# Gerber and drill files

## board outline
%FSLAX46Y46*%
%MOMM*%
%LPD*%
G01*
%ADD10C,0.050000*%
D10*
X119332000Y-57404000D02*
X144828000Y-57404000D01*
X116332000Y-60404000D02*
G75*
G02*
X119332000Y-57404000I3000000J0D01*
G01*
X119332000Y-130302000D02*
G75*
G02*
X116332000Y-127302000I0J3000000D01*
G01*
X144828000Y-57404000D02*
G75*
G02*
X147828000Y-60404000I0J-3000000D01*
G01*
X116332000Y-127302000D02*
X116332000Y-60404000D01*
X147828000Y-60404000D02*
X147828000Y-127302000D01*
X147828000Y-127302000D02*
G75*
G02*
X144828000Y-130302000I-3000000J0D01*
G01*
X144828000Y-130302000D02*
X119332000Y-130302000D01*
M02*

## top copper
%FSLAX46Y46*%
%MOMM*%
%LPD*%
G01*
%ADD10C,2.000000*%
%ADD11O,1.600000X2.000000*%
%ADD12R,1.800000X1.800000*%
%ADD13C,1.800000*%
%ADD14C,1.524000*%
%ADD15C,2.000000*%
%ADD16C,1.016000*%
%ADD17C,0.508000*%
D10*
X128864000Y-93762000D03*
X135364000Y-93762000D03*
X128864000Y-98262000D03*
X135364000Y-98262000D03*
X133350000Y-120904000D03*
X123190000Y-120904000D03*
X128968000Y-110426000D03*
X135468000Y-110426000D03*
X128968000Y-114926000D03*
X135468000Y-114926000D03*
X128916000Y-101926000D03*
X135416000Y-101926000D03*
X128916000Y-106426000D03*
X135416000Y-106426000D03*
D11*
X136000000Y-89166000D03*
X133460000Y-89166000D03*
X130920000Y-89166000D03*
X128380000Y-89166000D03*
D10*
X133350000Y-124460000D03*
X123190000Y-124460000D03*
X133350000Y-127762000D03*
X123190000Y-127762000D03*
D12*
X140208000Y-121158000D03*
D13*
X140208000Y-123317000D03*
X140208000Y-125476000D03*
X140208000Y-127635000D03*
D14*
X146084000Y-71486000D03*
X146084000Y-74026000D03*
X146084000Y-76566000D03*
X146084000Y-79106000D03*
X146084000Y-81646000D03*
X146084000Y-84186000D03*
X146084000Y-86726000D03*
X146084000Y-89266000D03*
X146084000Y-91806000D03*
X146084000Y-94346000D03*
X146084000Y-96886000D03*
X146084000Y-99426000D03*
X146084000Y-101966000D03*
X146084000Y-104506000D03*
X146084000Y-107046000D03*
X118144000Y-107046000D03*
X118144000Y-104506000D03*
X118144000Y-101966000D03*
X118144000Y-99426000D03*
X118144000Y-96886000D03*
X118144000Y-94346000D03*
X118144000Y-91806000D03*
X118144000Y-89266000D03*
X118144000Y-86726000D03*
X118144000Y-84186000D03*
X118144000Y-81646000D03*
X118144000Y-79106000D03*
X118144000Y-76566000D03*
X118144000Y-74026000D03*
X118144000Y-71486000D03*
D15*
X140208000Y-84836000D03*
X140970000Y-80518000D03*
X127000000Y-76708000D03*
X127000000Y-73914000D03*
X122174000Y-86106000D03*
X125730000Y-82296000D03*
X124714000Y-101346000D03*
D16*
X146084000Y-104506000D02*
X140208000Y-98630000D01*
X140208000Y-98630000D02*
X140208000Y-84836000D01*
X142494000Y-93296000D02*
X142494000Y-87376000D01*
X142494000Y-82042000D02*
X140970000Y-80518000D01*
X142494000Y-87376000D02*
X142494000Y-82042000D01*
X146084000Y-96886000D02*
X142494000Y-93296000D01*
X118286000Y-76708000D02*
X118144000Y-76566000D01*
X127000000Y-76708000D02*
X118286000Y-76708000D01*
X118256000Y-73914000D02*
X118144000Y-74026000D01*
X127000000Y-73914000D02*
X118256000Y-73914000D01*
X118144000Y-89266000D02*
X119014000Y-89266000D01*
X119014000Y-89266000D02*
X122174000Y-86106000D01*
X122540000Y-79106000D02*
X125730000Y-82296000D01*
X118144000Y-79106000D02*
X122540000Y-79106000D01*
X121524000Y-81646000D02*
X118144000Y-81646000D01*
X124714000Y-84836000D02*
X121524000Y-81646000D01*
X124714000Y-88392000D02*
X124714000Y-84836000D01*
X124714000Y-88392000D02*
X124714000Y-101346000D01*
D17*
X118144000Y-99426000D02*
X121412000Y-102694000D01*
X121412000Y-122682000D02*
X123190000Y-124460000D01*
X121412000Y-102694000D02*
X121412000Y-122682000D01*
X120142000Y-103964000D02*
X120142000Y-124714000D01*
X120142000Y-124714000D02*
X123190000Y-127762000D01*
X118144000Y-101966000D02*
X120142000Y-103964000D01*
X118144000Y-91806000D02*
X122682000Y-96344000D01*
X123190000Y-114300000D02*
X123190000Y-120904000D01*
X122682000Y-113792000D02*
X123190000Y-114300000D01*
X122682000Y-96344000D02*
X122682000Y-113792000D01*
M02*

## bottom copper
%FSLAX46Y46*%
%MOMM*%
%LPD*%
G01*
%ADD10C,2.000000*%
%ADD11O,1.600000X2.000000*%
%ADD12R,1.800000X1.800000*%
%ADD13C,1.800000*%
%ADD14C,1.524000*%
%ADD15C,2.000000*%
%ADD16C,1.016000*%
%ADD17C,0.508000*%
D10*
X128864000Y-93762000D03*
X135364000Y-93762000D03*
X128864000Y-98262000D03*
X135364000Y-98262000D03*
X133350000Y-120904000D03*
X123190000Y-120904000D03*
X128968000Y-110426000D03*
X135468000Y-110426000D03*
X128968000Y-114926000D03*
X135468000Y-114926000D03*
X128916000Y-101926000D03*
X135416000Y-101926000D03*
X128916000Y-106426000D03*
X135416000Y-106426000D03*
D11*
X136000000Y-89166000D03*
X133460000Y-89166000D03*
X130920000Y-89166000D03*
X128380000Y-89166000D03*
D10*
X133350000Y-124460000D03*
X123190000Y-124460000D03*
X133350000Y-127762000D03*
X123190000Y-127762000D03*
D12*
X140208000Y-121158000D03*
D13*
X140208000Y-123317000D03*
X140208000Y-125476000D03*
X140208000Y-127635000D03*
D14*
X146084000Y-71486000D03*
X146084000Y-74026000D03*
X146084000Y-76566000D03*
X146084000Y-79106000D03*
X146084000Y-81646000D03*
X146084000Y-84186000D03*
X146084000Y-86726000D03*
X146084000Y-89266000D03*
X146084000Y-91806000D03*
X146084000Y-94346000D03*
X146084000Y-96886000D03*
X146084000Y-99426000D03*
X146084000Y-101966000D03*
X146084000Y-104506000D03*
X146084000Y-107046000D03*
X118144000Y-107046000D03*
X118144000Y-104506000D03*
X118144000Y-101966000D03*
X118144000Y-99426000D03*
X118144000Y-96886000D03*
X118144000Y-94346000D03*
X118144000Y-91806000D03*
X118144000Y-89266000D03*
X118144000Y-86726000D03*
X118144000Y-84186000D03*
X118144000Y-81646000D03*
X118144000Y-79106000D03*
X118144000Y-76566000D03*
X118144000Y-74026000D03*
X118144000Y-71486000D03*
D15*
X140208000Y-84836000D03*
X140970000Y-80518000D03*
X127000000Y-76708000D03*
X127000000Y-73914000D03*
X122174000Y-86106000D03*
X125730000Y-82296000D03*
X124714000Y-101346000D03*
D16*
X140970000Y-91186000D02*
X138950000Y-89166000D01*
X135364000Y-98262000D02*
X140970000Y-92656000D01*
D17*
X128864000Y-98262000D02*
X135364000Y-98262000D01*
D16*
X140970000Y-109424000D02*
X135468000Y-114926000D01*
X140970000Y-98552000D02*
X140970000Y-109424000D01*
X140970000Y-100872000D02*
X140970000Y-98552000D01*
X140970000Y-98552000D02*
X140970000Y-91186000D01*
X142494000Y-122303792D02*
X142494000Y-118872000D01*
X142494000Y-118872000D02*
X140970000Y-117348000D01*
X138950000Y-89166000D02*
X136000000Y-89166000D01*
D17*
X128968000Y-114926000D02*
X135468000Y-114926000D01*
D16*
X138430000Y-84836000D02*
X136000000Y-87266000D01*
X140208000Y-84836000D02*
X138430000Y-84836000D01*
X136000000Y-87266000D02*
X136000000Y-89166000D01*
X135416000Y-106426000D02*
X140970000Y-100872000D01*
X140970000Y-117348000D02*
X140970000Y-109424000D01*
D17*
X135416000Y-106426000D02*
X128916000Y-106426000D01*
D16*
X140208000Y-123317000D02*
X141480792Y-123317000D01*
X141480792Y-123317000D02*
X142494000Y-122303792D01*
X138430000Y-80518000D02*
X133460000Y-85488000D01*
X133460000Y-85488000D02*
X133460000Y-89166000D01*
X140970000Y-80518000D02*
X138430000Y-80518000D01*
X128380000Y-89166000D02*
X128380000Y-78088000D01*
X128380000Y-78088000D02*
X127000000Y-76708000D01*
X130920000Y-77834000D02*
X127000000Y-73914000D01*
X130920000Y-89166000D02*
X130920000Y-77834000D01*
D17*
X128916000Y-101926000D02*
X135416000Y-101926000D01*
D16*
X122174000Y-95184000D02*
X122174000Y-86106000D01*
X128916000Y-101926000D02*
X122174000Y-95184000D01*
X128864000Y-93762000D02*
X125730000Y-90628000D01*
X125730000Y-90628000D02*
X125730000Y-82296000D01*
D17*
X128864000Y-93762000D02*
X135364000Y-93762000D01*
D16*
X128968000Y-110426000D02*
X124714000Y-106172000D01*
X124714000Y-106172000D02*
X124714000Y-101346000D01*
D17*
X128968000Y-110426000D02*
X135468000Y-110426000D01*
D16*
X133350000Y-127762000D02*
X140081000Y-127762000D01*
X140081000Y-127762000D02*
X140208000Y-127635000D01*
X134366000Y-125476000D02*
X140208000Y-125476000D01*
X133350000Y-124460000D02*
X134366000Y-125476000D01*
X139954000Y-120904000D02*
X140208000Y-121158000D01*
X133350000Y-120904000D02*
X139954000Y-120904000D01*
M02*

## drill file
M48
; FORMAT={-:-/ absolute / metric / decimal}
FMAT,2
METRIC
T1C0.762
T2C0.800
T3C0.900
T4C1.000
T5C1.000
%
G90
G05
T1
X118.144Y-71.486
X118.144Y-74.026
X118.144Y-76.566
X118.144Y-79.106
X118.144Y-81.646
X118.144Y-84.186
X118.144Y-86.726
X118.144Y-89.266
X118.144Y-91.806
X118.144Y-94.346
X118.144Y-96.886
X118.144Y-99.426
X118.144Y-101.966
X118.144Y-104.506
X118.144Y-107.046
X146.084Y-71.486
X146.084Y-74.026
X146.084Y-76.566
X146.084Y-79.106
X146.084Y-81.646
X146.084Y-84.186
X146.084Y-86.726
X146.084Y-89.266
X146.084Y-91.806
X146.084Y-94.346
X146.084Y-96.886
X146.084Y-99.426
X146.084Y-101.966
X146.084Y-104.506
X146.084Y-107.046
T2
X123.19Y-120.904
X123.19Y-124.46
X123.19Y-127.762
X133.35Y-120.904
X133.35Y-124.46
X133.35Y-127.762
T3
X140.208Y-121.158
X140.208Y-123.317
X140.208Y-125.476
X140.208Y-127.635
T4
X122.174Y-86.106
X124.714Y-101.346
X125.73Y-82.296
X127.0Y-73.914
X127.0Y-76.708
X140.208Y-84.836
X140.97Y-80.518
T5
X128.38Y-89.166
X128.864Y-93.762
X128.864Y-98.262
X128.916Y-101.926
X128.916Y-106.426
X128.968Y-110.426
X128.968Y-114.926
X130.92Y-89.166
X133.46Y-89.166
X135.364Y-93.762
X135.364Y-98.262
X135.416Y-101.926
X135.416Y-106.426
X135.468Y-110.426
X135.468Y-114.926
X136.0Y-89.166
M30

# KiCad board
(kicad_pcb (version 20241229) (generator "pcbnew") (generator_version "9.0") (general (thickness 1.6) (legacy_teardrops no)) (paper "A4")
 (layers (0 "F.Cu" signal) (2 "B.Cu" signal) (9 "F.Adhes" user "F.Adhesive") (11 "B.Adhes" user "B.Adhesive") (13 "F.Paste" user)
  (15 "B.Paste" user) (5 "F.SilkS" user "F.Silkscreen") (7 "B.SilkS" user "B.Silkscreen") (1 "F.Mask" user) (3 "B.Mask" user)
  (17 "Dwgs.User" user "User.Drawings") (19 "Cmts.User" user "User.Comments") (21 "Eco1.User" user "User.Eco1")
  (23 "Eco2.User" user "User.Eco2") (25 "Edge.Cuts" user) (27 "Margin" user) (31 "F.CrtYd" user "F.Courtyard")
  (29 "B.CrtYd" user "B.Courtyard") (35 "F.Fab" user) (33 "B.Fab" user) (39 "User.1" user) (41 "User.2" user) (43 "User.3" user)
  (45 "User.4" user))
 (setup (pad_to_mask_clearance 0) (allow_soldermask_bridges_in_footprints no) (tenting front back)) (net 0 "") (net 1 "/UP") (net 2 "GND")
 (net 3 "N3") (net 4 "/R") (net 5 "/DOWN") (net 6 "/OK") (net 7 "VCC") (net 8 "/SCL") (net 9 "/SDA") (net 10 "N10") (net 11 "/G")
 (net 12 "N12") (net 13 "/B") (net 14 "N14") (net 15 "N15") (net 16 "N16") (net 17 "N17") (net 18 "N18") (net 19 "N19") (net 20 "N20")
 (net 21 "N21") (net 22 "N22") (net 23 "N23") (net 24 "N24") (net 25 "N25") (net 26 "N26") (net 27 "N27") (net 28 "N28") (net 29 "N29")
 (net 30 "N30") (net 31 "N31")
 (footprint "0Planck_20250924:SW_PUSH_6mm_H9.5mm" (layer "F.Cu") (at 128.864 93.762)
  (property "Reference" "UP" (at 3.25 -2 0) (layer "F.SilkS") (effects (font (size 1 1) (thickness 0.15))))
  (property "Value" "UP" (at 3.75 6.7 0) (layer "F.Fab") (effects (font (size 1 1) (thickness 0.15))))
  (pad "1" thru_hole circle (at 0 0) (size 2 2) (drill 1) (layers "*.Cu" "*.Mask") (remove_unused_layers no) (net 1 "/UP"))
  (pad "1" thru_hole circle (at 6.5 0) (size 2 2) (drill 1) (layers "*.Cu" "*.Mask") (remove_unused_layers no) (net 1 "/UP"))
  (pad "2" thru_hole circle (at 0 4.5) (size 2 2) (drill 1) (layers "*.Cu" "*.Mask") (remove_unused_layers no) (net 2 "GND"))
  (pad "2" thru_hole circle (at 6.5 4.5) (size 2 2) (drill 1) (layers "*.Cu" "*.Mask") (remove_unused_layers no) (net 2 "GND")))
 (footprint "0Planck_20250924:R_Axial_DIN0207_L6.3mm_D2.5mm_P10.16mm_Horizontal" (layer "F.Cu") (at 133.35 120.904 180)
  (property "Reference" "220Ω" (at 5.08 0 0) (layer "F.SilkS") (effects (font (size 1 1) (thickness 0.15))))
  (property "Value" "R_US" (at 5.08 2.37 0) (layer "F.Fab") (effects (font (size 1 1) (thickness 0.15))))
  (pad "1" thru_hole circle (at 0 0 180) (size 2 2) (drill 0.8) (layers "*.Cu" "*.Mask") (remove_unused_layers no) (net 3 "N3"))
  (pad "2" thru_hole circle (at 10.16 0 180) (size 2 2) (drill 0.8) (layers "*.Cu" "*.Mask") (remove_unused_layers no) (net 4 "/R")))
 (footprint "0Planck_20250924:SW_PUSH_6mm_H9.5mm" (layer "F.Cu") (at 128.968 110.426)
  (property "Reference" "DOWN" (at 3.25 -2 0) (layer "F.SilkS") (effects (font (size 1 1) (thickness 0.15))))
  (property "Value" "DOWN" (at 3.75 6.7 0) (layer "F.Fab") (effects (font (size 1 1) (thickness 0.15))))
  (pad "1" thru_hole circle (at 0 0) (size 2 2) (drill 1) (layers "*.Cu" "*.Mask") (remove_unused_layers no) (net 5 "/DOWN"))
  (pad "1" thru_hole circle (at 6.5 0) (size 2 2) (drill 1) (layers "*.Cu" "*.Mask") (remove_unused_layers no) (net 5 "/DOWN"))
  (pad "2" thru_hole circle (at 0 4.5) (size 2 2) (drill 1) (layers "*.Cu" "*.Mask") (remove_unused_layers no) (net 2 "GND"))
  (pad "2" thru_hole circle (at 6.5 4.5) (size 2 2) (drill 1) (layers "*.Cu" "*.Mask") (remove_unused_layers no) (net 2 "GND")))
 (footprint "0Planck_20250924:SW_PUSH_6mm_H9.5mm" (layer "F.Cu") (at 128.916 101.926)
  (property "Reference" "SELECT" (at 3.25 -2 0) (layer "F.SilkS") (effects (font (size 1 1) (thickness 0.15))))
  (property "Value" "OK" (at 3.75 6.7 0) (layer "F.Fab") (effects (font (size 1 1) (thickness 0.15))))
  (pad "1" thru_hole circle (at 0 0) (size 2 2) (drill 1) (layers "*.Cu" "*.Mask") (remove_unused_layers no) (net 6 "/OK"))
  (pad "1" thru_hole circle (at 6.5 0) (size 2 2) (drill 1) (layers "*.Cu" "*.Mask") (remove_unused_layers no) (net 6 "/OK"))
  (pad "2" thru_hole circle (at 0 4.5) (size 2 2) (drill 1) (layers "*.Cu" "*.Mask") (remove_unused_layers no) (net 2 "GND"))
  (pad "2" thru_hole circle (at 6.5 4.5) (size 2 2) (drill 1) (layers "*.Cu" "*.Mask") (remove_unused_layers no) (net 2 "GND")))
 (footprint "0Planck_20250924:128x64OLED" (layer "F.Cu") (at 132.38 78.566 180)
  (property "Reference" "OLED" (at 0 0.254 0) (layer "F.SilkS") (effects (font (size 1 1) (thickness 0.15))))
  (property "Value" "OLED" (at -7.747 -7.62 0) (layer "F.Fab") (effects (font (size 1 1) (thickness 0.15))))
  (pad "1" thru_hole oval (at -3.62 -10.6 270) (size 2 1.6) (drill 1) (layers "*.Cu" "*.Mask") (remove_unused_layers no) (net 2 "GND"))
  (pad "2" thru_hole oval (at -1.08 -10.6 270) (size 2 1.6) (drill 1) (layers "*.Cu" "*.Mask") (remove_unused_layers no) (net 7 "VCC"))
  (pad "3" thru_hole oval (at 1.46 -10.6 270) (size 2 1.6) (drill 1) (layers "*.Cu" "*.Mask") (remove_unused_layers no) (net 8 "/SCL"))
  (pad "4" thru_hole oval (at 4 -10.6 270) (size 2 1.6) (drill 1) (layers "*.Cu" "*.Mask") (remove_unused_layers no) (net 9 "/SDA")))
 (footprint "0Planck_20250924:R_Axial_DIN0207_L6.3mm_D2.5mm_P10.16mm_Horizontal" (layer "F.Cu") (at 133.35 124.46 180)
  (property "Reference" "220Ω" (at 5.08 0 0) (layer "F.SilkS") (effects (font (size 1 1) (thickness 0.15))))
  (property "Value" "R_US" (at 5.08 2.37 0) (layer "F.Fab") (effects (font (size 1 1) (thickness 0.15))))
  (pad "1" thru_hole circle (at 0 0 180) (size 2 2) (drill 0.8) (layers "*.Cu" "*.Mask") (remove_unused_layers no) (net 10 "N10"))
  (pad "2" thru_hole circle (at 10.16 0 180) (size 2 2) (drill 0.8) (layers "*.Cu" "*.Mask") (remove_unused_layers no) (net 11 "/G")))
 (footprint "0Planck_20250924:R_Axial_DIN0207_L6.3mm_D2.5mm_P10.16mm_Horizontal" (layer "F.Cu") (at 133.35 127.762 180)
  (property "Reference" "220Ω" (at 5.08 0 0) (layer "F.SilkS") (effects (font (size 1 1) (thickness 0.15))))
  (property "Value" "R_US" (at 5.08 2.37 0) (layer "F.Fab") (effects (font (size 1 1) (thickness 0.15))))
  (pad "1" thru_hole circle (at 0 0 180) (size 2 2) (drill 0.8) (layers "*.Cu" "*.Mask") (remove_unused_layers no) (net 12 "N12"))
  (pad "2" thru_hole circle (at 10.16 0 180) (size 2 2) (drill 0.8) (layers "*.Cu" "*.Mask") (remove_unused_layers no) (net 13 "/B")))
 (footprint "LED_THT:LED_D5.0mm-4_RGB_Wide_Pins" (layer "F.Cu") (at 140.208 121.158 -90)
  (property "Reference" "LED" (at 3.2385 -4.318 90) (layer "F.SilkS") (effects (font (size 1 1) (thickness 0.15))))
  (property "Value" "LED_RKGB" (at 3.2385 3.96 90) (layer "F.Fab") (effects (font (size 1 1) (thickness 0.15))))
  (pad "1" thru_hole rect (at 0 0 270) (size 1.8 1.8) (drill 0.9) (layers "*.Cu" "*.Mask") (remove_unused_layers no) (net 3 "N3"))
  (pad "2" thru_hole circle (at 2.159 0 270) (size 1.8 1.8) (drill 0.9) (layers "*.Cu" "*.Mask") (remove_unused_layers no) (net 2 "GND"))
  (pad "3" thru_hole circle (at 4.318 0 270) (size 1.8 1.8) (drill 0.9) (layers "*.Cu" "*.Mask") (remove_unused_layers no) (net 10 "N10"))
  (pad "4" thru_hole circle (at 6.477 0 270) (size 1.8 1.8) (drill 0.9) (layers "*.Cu" "*.Mask") (remove_unused_layers no) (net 12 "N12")))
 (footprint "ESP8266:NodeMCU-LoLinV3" (layer "B.Cu") (at 132.114 91.806 180)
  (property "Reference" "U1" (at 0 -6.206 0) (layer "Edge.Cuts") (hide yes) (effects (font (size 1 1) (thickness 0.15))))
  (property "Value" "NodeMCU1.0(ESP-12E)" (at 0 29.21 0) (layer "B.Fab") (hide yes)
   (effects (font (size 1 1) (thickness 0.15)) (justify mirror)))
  (pad "1" thru_hole circle (at -13.97 20.32 180) (size 1.524 1.524) (drill 0.762) (layers "*.Cu" "*.Mask" "B.SilkS")
   (remove_unused_layers no) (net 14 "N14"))
  (pad "2" thru_hole circle (at -13.97 17.78 180) (size 1.524 1.524) (drill 0.762) (layers "*.Cu" "*.Mask" "B.SilkS")
   (remove_unused_layers no) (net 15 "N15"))
  (pad "3" thru_hole circle (at -13.97 15.24 180) (size 1.524 1.524) (drill 0.762) (layers "*.Cu" "*.Mask" "B.SilkS")
   (remove_unused_layers no) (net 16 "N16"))
  (pad "4" thru_hole circle (at -13.97 12.7 180) (size 1.524 1.524) (drill 0.762) (layers "*.Cu" "*.Mask" "B.SilkS")
   (remove_unused_layers no) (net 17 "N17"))
  (pad "5" thru_hole circle (at -13.97 10.16 180) (size 1.524 1.524) (drill 0.762) (layers "*.Cu" "*.Mask" "B.SilkS")
   (remove_unused_layers no) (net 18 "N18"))
  (pad "6" thru_hole circle (at -13.97 7.62 180) (size 1.524 1.524) (drill 0.762) (layers "*.Cu" "*.Mask" "B.SilkS")
   (remove_unused_layers no) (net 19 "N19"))
  (pad "7" thru_hole circle (at -13.97 5.08 180) (size 1.524 1.524) (drill 0.762) (layers "*.Cu" "*.Mask" "B.SilkS")
   (remove_unused_layers no) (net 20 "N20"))
  (pad "8" thru_hole circle (at -13.97 2.54 180) (size 1.524 1.524) (drill 0.762) (layers "*.Cu" "*.Mask" "B.SilkS")
   (remove_unused_layers no) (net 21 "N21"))
  (pad "9" thru_hole circle (at -13.97 0 180) (size 1.524 1.524) (drill 0.762) (layers "*.Cu" "*.Mask" "B.SilkS") (remove_unused_layers no)
   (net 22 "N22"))
  (pad "10" thru_hole circle (at -13.97 -2.54 180) (size 1.524 1.524) (drill 0.762) (layers "*.Cu" "*.Mask" "B.SilkS")
   (remove_unused_layers no) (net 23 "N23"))
  (pad "11" thru_hole circle (at -13.97 -5.08 180) (size 1.524 1.524) (drill 0.762) (layers "*.Cu" "*.Mask" "B.SilkS")
   (remove_unused_layers no) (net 7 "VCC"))
  (pad "12" thru_hole circle (at -13.97 -7.62 180) (size 1.524 1.524) (drill 0.762) (layers "*.Cu" "*.Mask" "B.SilkS")
   (remove_unused_layers no) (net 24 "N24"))
  (pad "13" thru_hole circle (at -13.97 -10.16 180) (size 1.524 1.524) (drill 0.762) (layers "*.Cu" "*.Mask" "B.SilkS")
   (remove_unused_layers no) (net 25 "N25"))
  (pad "14" thru_hole circle (at -13.97 -12.7 180) (size 1.524 1.524) (drill 0.762) (layers "*.Cu" "*.Mask" "B.SilkS")
   (remove_unused_layers no) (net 2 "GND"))
  (pad "15" thru_hole circle (at -13.97 -15.24 180) (size 1.524 1.524) (drill 0.762) (layers "*.Cu" "*.Mask" "B.SilkS")
   (remove_unused_layers no) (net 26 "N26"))
  (pad "16" thru_hole circle (at 13.97 -15.24 180) (size 1.524 1.524) (drill 0.762) (layers "*.Cu" "*.Mask" "B.SilkS")
   (remove_unused_layers no) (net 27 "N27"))
  (pad "17" thru_hole circle (at 13.97 -12.7 180) (size 1.524 1.524) (drill 0.762) (layers "*.Cu" "*.Mask" "B.SilkS")
   (remove_unused_layers no) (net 2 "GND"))
  (pad "18" thru_hole circle (at 13.97 -10.16 180) (size 1.524 1.524) (drill 0.762) (layers "*.Cu" "*.Mask" "B.SilkS")
   (remove_unused_layers no) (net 13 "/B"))
  (pad "19" thru_hole circle (at 13.97 -7.62 180) (size 1.524 1.524) (drill 0.762) (layers "*.Cu" "*.Mask" "B.SilkS")
   (remove_unused_layers no) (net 11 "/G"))
  (pad "20" thru_hole circle (at 13.97 -5.08 180) (size 1.524 1.524) (drill 0.762) (layers "*.Cu" "*.Mask" "B.SilkS")
   (remove_unused_layers no) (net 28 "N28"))
  (pad "21" thru_hole circle (at 13.97 -2.54 180) (size 1.524 1.524) (drill 0.762) (layers "*.Cu" "*.Mask" "B.SilkS")
   (remove_unused_layers no) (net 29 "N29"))
  (pad "22" thru_hole circle (at 13.97 0 180) (size 1.524 1.524) (drill 0.762) (layers "*.Cu" "*.Mask" "B.SilkS") (remove_unused_layers no)
   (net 4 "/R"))
  (pad "23" thru_hole circle (at 13.97 2.54 180) (size 1.524 1.524) (drill 0.762) (layers "*.Cu" "*.Mask" "B.SilkS")
   (remove_unused_layers no) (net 6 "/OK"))
  (pad "24" thru_hole circle (at 13.97 5.08 180) (size 1.524 1.524) (drill 0.762) (layers "*.Cu" "*.Mask" "B.SilkS")
   (remove_unused_layers no) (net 2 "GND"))
  (pad "25" thru_hole circle (at 13.97 7.62 180) (size 1.524 1.524) (drill 0.762) (layers "*.Cu" "*.Mask" "B.SilkS")
   (remove_unused_layers no) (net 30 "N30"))
  (pad "26" thru_hole circle (at 13.97 10.16 180) (size 1.524 1.524) (drill 0.762) (layers "*.Cu" "*.Mask" "B.SilkS")
   (remove_unused_layers no) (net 5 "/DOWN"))
  (pad "27" thru_hole circle (at 13.97 12.7 180) (size 1.524 1.524) (drill 0.762) (layers "*.Cu" "*.Mask" "B.SilkS")
   (remove_unused_layers no) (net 1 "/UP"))
  (pad "28" thru_hole circle (at 13.97 15.24 180) (size 1.524 1.524) (drill 0.762) (layers "*.Cu" "*.Mask" "B.SilkS")
   (remove_unused_layers no) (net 9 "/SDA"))
  (pad "29" thru_hole circle (at 13.97 17.78 180) (size 1.524 1.524) (drill 0.762) (layers "*.Cu" "*.Mask" "B.SilkS")
   (remove_unused_layers no) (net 8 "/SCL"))
  (pad "30" thru_hole circle (at 13.97 20.32 180) (size 1.524 1.524) (drill 0.762) (layers "*.Cu" "*.Mask" "B.SilkS")
   (remove_unused_layers no) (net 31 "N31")))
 (gr_line (start 119.332 57.404) (end 144.828 57.404) (stroke (width 0.05) (type default)) (layer "Edge.Cuts"))
 (gr_arc (start 116.332 60.404) (mid 117.21068 58.28268) (end 119.332 57.404) (stroke (width 0.05) (type default)) (layer "Edge.Cuts"))
 (gr_arc (start 119.332 130.302) (mid 117.21068 129.42332) (end 116.332 127.302) (stroke (width 0.05) (type default)) (layer "Edge.Cuts"))
 (gr_arc (start 144.828 57.404) (mid 146.94932 58.28268) (end 147.828 60.404) (stroke (width 0.05) (type default)) (layer "Edge.Cuts"))
 (gr_line (start 116.332 127.302) (end 116.332 60.404) (stroke (width 0.05) (type default)) (layer "Edge.Cuts"))
 (gr_line (start 147.828 60.404) (end 147.828 127.302) (stroke (width 0.05) (type default)) (layer "Edge.Cuts"))
 (gr_arc (start 147.828 127.302) (mid 146.94932 129.42332) (end 144.828 130.302) (stroke (width 0.05) (type default)) (layer "Edge.Cuts"))
 (gr_line (start 144.828 130.302) (end 119.332 130.302) (stroke (width 0.05) (type default)) (layer "Edge.Cuts"))
 (segment (start 146.084 104.506) (end 140.208 98.63) (width 1.016) (layer "F.Cu") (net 2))
 (segment (start 140.208 98.63) (end 140.208 84.836) (width 1.016) (layer "F.Cu") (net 2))
 (via (at 140.208 84.836) (size 2) (drill 1) (layers "F.Cu" "B.Cu") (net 2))
 (segment (start 140.97 91.186) (end 138.95 89.166) (width 1.016) (layer "B.Cu") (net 2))
 (segment (start 135.364 98.262) (end 140.97 92.656) (width 1.016) (layer "B.Cu") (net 2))
 (segment (start 128.864 98.262) (end 135.364 98.262) (width 0.508) (layer "B.Cu") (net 2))
 (segment (start 140.97 109.424) (end 135.468 114.926) (width 1.016) (layer "B.Cu") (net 2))
 (segment (start 140.97 98.552) (end 140.97 109.424) (width 1.016) (layer "B.Cu") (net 2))
 (segment (start 140.97 100.872) (end 140.97 98.552) (width 1.016) (layer "B.Cu") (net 2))
 (segment (start 140.97 98.552) (end 140.97 91.186) (width 1.016) (layer "B.Cu") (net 2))
 (segment (start 142.494 122.303792) (end 142.494 118.872) (width 1.016) (layer "B.Cu") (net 2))
 (segment (start 142.494 118.872) (end 140.97 117.348) (width 1.016) (layer "B.Cu") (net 2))
 (segment (start 138.95 89.166) (end 136 89.166) (width 1.016) (layer "B.Cu") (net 2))
 (segment (start 128.968 114.926) (end 135.468 114.926) (width 0.508) (layer "B.Cu") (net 2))
 (segment (start 138.43 84.836) (end 136 87.266) (width 1.016) (layer "B.Cu") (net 2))
 (segment (start 140.208 84.836) (end 138.43 84.836) (width 1.016) (layer "B.Cu") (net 2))
 (segment (start 136 87.266) (end 136 89.166) (width 1.016) (layer "B.Cu") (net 2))
 (segment (start 135.416 106.426) (end 140.97 100.872) (width 1.016) (layer "B.Cu") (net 2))
 (segment (start 140.97 117.348) (end 140.97 109.424) (width 1.016) (layer "B.Cu") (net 2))
 (segment (start 135.416 106.426) (end 128.916 106.426) (width 0.508) (layer "B.Cu") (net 2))
 (segment (start 140.208 123.317) (end 141.480792 123.317) (width 1.016) (layer "B.Cu") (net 2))
 (segment (start 141.480792 123.317) (end 142.494 122.303792) (width 1.016) (layer "B.Cu") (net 2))
 (segment (start 142.494 93.296) (end 142.494 87.376) (width 1.016) (layer "F.Cu") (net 7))
 (segment (start 142.494 82.042) (end 140.97 80.518) (width 1.016) (layer "F.Cu") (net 7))
 (segment (start 142.494 87.376) (end 142.494 82.042) (width 1.016) (layer "F.Cu") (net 7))
 (segment (start 146.084 96.886) (end 142.494 93.296) (width 1.016) (layer "F.Cu") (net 7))
 (via (at 140.97 80.518) (size 2) (drill 1) (layers "F.Cu" "B.Cu") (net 7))
 (segment (start 138.43 80.518) (end 133.46 85.488) (width 1.016) (layer "B.Cu") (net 7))
 (segment (start 133.46 85.488) (end 133.46 89.166) (width 1.016) (layer "B.Cu") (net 7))
 (segment (start 140.97 80.518) (end 138.43 80.518) (width 1.016) (layer "B.Cu") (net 7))
 (segment (start 118.286 76.708) (end 118.144 76.566) (width 1.016) (layer "F.Cu") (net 9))
 (segment (start 127 76.708) (end 118.286 76.708) (width 1.016) (layer "F.Cu") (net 9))
 (via (at 127 76.708) (size 2) (drill 1) (layers "F.Cu" "B.Cu") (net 9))
 (segment (start 128.38 89.166) (end 128.38 78.088) (width 1.016) (layer "B.Cu") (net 9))
 (segment (start 128.38 78.088) (end 127 76.708) (width 1.016) (layer "B.Cu") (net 9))
 (segment (start 118.256 73.914) (end 118.144 74.026) (width 1.016) (layer "F.Cu") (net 8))
 (segment (start 127 73.914) (end 118.256 73.914) (width 1.016) (layer "F.Cu") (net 8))
 (via (at 127 73.914) (size 2) (drill 1) (layers "F.Cu" "B.Cu") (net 8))
 (segment (start 130.92 77.834) (end 127 73.914) (width 1.016) (layer "B.Cu") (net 8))
 (segment (start 130.92 89.166) (end 130.92 77.834) (width 1.016) (layer "B.Cu") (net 8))
 (segment (start 118.144 89.266) (end 119.014 89.266) (width 1.016) (layer "F.Cu") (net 6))
 (segment (start 119.014 89.266) (end 122.174 86.106) (width 1.016) (layer "F.Cu") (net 6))
 (via (at 122.174 86.106) (size 2) (drill 1) (layers "F.Cu" "B.Cu") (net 6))
 (segment (start 128.916 101.926) (end 135.416 101.926) (width 0.508) (layer "B.Cu") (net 6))
 (segment (start 122.174 95.184) (end 122.174 86.106) (width 1.016) (layer "B.Cu") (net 6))
 (segment (start 128.916 101.926) (end 122.174 95.184) (width 1.016) (layer "B.Cu") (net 6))
 (segment (start 122.54 79.106) (end 125.73 82.296) (width 1.016) (layer "F.Cu") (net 1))
 (segment (start 118.144 79.106) (end 122.54 79.106) (width 1.016) (layer "F.Cu") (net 1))
 (via (at 125.73 82.296) (size 2) (drill 1) (layers "F.Cu" "B.Cu") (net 1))
 (segment (start 128.864 93.762) (end 125.73 90.628) (width 1.016) (layer "B.Cu") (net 1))
 (segment (start 125.73 90.628) (end 125.73 82.296) (width 1.016) (layer "B.Cu") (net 1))
 (segment (start 128.864 93.762) (end 135.364 93.762) (width 0.508) (layer "B.Cu") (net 1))
 (segment (start 121.524 81.646) (end 118.144 81.646) (width 1.016) (layer "F.Cu") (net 5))
 (segment (start 124.714 84.836) (end 121.524 81.646) (width 1.016) (layer "F.Cu") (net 5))
 (segment (start 124.714 88.392) (end 124.714 84.836) (width 1.016) (layer "F.Cu") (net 5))
 (segment (start 124.714 88.392) (end 124.714 101.346) (width 1.016) (layer "F.Cu") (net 5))
 (via (at 124.714 101.346) (size 2) (drill 1) (layers "F.Cu" "B.Cu") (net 5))
 (segment (start 128.968 110.426) (end 124.714 106.172) (width 1.016) (layer "B.Cu") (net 5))
 (segment (start 124.714 106.172) (end 124.714 101.346) (width 1.016) (layer "B.Cu") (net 5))
 (segment (start 128.968 110.426) (end 135.468 110.426) (width 0.508) (layer "B.Cu") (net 5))
 (segment (start 118.144 99.426) (end 121.412 102.694) (width 0.508) (layer "F.Cu") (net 11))
 (segment (start 121.412 122.682) (end 123.19 124.46) (width 0.508) (layer "F.Cu") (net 11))
 (segment (start 121.412 102.694) (end 121.412 122.682) (width 0.508) (layer "F.Cu") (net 11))
 (segment (start 120.142 103.964) (end 120.142 124.714) (width 0.508) (layer "F.Cu") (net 13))
 (segment (start 120.142 124.714) (end 123.19 127.762) (width 0.508) (layer "F.Cu") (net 13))
 (segment (start 118.144 101.966) (end 120.142 103.964) (width 0.508) (layer "F.Cu") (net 13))
 (segment (start 118.144 91.806) (end 122.682 96.344) (width 0.508) (layer "F.Cu") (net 4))
 (segment (start 123.19 114.3) (end 123.19 120.904) (width 0.508) (layer "F.Cu") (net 4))
 (segment (start 122.682 113.792) (end 123.19 114.3) (width 0.508) (layer "F.Cu") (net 4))
 (segment (start 122.682 96.344) (end 122.682 113.792) (width 0.508) (layer "F.Cu") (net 4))
 (segment (start 133.35 127.762) (end 140.081 127.762) (width 1.016) (layer "B.Cu") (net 12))
 (segment (start 140.081 127.762) (end 140.208 127.635) (width 1.016) (layer "B.Cu") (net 12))
 (segment (start 134.366 125.476) (end 140.208 125.476) (width 1.016) (layer "B.Cu") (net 10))
 (segment (start 133.35 124.46) (end 134.366 125.476) (width 1.016) (layer "B.Cu") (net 10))
 (segment (start 139.954 120.904) (end 140.208 121.158) (width 1.016) (layer "B.Cu") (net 3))
 (segment (start 133.35 120.904) (end 139.954 120.904) (width 1.016) (layer "B.Cu") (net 3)))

